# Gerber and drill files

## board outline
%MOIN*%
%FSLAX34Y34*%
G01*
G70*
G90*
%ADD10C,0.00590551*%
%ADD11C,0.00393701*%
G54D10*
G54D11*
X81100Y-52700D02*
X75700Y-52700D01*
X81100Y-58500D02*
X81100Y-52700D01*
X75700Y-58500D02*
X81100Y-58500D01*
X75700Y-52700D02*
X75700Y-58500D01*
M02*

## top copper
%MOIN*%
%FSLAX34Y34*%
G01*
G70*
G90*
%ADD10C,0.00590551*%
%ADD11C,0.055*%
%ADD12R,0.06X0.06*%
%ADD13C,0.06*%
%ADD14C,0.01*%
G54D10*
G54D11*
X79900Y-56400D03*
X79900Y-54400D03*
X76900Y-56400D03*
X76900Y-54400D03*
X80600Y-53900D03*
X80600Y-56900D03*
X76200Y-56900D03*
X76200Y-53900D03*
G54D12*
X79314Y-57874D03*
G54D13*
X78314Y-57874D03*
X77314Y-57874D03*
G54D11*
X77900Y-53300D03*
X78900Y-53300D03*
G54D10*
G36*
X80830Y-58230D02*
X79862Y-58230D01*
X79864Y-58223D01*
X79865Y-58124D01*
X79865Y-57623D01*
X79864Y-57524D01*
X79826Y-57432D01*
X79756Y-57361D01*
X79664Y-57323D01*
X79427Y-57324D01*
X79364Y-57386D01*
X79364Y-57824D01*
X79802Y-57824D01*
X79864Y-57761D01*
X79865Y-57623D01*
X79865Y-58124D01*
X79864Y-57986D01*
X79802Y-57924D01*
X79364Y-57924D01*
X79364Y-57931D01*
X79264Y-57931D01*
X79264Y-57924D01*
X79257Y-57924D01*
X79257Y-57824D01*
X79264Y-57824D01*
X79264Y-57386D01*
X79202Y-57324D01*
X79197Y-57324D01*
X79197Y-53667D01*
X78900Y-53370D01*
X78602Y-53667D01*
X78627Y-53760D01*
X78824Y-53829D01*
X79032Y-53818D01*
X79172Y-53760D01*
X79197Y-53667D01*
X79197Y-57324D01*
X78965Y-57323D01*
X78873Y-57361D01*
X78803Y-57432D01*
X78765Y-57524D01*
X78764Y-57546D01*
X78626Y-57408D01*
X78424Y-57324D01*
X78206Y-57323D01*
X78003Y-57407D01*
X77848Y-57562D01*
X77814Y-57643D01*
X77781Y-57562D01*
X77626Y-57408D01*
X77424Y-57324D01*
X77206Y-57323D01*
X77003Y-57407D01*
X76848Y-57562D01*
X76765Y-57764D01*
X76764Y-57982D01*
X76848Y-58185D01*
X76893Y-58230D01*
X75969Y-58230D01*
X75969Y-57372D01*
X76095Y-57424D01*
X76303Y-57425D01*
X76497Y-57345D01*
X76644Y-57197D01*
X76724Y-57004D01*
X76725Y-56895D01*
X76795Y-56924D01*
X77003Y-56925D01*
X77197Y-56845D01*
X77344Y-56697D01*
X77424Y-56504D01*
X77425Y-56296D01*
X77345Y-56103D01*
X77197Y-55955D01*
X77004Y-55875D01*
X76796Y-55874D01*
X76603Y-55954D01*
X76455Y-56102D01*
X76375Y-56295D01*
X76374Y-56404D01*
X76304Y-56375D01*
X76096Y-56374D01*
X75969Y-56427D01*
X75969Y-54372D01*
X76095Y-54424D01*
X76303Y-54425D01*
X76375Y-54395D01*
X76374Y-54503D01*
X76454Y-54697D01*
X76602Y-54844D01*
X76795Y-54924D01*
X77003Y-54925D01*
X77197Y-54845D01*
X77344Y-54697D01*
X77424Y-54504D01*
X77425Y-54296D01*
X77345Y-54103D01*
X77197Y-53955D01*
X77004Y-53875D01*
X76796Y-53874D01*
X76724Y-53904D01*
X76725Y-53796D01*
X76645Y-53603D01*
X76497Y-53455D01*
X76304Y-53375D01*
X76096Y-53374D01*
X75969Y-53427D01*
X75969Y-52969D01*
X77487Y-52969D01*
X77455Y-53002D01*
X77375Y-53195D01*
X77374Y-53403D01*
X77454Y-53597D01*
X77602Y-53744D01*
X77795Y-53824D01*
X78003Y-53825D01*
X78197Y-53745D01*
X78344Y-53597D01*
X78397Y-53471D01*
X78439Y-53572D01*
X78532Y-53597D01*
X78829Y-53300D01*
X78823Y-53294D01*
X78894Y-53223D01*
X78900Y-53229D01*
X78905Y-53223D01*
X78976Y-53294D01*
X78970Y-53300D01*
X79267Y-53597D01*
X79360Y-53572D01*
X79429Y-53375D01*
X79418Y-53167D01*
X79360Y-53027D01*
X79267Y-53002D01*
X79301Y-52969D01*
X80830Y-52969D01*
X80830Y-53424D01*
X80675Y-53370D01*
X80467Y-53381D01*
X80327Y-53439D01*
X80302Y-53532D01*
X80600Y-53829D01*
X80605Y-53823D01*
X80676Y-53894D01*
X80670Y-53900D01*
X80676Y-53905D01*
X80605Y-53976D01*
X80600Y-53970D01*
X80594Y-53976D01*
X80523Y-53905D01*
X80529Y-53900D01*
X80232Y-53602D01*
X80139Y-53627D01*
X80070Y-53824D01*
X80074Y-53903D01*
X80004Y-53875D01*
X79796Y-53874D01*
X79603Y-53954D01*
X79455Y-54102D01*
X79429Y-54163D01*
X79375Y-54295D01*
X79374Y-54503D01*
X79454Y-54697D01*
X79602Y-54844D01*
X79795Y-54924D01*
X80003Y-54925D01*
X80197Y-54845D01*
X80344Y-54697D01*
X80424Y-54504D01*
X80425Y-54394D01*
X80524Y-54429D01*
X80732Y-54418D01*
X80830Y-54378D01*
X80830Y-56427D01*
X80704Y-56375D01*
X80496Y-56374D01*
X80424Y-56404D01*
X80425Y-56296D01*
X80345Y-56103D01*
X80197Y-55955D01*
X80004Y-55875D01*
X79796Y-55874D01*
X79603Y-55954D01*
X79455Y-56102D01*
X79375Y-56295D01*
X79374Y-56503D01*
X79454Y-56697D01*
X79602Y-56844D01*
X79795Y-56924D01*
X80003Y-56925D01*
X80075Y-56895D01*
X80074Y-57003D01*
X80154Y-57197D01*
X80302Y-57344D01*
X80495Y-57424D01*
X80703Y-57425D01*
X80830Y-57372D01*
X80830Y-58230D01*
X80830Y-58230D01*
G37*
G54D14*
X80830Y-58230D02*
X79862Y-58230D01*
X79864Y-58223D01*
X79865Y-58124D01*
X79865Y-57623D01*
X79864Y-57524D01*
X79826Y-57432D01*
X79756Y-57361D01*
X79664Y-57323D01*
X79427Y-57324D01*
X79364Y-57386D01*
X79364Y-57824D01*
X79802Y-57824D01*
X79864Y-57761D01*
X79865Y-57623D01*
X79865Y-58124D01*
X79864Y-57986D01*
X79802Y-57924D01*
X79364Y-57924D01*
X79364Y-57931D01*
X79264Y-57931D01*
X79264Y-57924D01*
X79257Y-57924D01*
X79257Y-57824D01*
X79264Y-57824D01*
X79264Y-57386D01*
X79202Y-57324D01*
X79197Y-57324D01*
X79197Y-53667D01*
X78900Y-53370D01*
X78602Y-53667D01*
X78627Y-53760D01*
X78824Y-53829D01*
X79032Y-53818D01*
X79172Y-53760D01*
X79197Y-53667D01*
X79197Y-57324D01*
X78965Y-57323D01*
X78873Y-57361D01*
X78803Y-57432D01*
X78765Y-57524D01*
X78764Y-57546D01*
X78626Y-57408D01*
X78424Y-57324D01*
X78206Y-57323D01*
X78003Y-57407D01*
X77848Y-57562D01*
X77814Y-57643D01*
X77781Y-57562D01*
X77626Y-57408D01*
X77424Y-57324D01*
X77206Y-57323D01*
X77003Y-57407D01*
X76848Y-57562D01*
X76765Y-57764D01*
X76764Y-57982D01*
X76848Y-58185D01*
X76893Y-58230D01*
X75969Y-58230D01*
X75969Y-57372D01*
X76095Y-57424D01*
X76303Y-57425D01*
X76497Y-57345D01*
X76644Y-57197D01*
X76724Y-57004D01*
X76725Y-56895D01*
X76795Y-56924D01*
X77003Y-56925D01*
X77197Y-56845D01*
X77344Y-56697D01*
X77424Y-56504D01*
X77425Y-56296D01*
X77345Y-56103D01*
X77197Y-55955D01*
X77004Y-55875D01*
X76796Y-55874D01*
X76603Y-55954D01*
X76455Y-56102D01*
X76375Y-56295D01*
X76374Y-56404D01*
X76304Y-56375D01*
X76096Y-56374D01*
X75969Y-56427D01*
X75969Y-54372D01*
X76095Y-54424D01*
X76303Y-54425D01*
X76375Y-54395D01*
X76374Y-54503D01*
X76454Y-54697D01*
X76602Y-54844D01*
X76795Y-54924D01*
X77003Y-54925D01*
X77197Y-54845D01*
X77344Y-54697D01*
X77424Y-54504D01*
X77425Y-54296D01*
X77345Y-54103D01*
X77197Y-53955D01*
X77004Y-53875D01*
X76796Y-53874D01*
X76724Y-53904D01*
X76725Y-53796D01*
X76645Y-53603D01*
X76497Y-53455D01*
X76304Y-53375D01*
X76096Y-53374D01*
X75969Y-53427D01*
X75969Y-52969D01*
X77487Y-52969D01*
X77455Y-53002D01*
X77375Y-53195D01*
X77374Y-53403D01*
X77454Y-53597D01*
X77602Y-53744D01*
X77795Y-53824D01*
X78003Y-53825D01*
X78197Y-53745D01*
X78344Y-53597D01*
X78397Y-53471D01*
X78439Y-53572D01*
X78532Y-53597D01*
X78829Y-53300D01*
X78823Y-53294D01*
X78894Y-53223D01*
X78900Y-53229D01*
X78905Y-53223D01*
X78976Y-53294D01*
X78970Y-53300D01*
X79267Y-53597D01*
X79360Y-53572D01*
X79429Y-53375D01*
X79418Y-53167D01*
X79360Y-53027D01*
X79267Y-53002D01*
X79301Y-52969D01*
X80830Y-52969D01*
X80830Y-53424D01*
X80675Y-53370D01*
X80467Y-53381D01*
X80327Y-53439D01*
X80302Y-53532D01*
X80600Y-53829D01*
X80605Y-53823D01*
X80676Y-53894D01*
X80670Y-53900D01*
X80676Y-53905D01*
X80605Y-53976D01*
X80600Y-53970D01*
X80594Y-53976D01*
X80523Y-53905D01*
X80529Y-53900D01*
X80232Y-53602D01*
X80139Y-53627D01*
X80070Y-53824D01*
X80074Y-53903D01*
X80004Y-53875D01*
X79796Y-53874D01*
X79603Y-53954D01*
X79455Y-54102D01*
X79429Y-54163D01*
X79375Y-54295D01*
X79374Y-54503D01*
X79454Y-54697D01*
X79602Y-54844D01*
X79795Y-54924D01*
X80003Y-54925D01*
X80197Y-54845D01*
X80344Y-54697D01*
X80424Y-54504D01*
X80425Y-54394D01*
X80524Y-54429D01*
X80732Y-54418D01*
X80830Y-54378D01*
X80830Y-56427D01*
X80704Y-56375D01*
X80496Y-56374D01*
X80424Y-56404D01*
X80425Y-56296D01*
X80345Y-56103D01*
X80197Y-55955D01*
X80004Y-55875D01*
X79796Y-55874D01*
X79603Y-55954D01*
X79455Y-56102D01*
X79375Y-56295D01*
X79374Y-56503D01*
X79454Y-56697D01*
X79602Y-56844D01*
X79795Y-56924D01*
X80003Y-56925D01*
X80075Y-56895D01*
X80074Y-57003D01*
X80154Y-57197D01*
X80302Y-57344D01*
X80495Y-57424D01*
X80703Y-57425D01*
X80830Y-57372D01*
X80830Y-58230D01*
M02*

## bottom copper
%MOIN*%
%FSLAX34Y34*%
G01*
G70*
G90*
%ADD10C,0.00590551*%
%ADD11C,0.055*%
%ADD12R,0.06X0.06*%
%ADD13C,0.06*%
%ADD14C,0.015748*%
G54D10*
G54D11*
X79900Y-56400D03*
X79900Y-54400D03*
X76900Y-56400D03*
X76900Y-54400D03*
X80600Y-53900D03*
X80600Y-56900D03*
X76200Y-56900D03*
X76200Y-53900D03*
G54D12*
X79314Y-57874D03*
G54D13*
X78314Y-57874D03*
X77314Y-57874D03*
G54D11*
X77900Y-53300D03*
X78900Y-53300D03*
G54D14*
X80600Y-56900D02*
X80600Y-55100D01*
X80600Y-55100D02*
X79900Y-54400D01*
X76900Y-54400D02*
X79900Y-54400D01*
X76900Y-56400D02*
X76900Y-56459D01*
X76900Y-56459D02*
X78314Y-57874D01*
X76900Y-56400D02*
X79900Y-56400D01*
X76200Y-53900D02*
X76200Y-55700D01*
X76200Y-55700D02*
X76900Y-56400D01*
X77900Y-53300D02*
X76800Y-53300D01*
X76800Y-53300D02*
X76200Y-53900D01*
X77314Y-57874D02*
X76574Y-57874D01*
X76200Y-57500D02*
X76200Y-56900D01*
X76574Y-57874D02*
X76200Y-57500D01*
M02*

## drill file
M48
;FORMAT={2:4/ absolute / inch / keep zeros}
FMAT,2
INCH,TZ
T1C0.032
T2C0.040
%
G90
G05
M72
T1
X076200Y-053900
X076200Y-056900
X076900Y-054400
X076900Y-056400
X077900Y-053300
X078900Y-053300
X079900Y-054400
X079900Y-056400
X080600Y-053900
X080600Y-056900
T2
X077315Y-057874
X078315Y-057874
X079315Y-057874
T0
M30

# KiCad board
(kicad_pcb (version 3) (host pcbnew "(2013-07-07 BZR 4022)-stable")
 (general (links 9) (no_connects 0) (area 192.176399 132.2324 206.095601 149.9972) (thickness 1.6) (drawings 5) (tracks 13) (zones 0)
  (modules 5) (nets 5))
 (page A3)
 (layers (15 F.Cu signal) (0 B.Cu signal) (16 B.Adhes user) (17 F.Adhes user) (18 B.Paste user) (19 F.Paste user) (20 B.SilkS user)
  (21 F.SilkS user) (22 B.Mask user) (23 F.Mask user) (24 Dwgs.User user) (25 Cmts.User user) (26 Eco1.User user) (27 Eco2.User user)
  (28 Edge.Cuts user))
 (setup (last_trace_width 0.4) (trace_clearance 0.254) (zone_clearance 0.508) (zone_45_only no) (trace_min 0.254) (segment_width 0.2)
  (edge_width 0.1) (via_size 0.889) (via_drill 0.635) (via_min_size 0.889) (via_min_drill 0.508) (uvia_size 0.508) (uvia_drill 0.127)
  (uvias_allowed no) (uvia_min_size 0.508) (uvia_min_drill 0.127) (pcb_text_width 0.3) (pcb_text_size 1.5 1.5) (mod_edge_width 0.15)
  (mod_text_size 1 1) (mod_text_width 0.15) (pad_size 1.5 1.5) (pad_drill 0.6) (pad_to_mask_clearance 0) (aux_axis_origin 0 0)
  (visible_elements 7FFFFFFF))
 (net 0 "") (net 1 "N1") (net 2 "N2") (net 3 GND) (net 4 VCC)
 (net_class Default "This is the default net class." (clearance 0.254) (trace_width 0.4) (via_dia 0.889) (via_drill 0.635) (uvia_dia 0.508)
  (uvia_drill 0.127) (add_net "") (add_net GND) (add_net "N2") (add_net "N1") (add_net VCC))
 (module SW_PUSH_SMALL (layer B.Cu) (at 199.136 140.716)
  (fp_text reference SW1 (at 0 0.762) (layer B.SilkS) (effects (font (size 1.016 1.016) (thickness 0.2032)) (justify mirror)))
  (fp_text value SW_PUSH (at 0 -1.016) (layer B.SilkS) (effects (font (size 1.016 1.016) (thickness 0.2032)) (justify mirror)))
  (pad 1 thru_hole circle (at 3.81 2.54) (size 1.397 1.397) (drill 0.8128) (layers *.Cu *.Mask B.SilkS) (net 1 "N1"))
  (pad 2 thru_hole circle (at 3.81 -2.54) (size 1.397 1.397) (drill 0.8128) (layers *.Cu *.Mask B.SilkS) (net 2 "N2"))
  (pad 1 thru_hole circle (at -3.81 2.54) (size 1.397 1.397) (drill 0.8128) (layers *.Cu *.Mask B.SilkS) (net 1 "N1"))
  (pad 2 thru_hole circle (at -3.81 -2.54) (size 1.397 1.397) (drill 0.8128) (layers *.Cu *.Mask B.SilkS) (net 2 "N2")))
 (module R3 (layer F.Cu) (at 204.724 140.716 270) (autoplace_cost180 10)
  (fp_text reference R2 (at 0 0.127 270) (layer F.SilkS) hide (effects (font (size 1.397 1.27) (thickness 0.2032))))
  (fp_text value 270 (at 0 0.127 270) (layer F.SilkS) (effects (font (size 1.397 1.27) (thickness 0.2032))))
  (pad 1 thru_hole circle (at -3.81 0 270) (size 1.397 1.397) (drill 0.8128) (layers *.Cu *.Mask F.SilkS) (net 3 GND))
  (pad 2 thru_hole circle (at 3.81 0 270) (size 1.397 1.397) (drill 0.8128) (layers *.Cu *.Mask F.SilkS) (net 2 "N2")))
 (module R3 (layer F.Cu) (at 193.548 140.716 90) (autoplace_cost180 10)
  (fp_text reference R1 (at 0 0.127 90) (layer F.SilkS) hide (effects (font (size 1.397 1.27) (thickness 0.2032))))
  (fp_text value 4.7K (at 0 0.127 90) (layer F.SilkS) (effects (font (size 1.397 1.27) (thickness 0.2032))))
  (pad 1 thru_hole circle (at -3.81 0 90) (size 1.397 1.397) (drill 0.8128) (layers *.Cu *.Mask F.SilkS) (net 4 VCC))
  (pad 2 thru_hole circle (at 3.81 0 90) (size 1.397 1.397) (drill 0.8128) (layers *.Cu *.Mask F.SilkS) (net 1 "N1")))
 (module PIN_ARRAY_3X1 (layer F.Cu) (at 198.92 147 180)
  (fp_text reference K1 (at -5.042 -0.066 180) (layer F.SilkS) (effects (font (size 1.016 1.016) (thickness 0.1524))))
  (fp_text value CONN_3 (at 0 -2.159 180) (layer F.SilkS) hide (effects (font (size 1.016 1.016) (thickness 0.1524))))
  (pad 1 thru_hole rect (at -2.54 0 180) (size 1.524 1.524) (drill 1.016) (layers *.Cu *.Mask F.SilkS) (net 3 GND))
  (pad 2 thru_hole circle (at 0 0 180) (size 1.524 1.524) (drill 1.016) (layers *.Cu *.Mask F.SilkS) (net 1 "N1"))
  (pad 3 thru_hole circle (at 2.54 0 180) (size 1.524 1.524) (drill 1.016) (layers *.Cu *.Mask F.SilkS) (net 4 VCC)))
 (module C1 (layer F.Cu) (at 199.136 135.382)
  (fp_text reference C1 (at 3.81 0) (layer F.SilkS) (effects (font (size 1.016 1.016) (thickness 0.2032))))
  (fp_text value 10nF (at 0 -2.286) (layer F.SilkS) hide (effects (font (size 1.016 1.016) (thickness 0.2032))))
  (pad 1 thru_hole circle (at -1.27 0) (size 1.397 1.397) (drill 0.8128) (layers *.Cu *.Mask F.SilkS) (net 1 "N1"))
  (pad 2 thru_hole circle (at 1.27 0) (size 1.397 1.397) (drill 0.8128) (layers *.Cu *.Mask F.SilkS) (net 3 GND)))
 (gr_line (start 205.994 133.858) (end 192.278 133.858) (angle 90) (layer Edge.Cuts) (width 0.1))
 (gr_line (start 205.994 148.59) (end 205.994 133.858) (angle 90) (layer Edge.Cuts) (width 0.1))
 (gr_line (start 192.278 148.59) (end 205.994 148.59) (angle 90) (layer Edge.Cuts) (width 0.1))
 (gr_line (start 192.278 133.858) (end 192.278 148.59) (angle 90) (layer Edge.Cuts) (width 0.1))
 (segment (start 204.724 144.526) (end 204.724 139.954) (width 0.4) (layer B.Cu) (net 2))
 (segment (start 204.724 139.954) (end 202.946 138.176) (width 0.4) (layer B.Cu) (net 2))
 (segment (start 195.326 138.176) (end 202.946 138.176) (width 0.4) (layer B.Cu) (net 2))
 (segment (start 195.326 143.256) (end 195.326 143.406) (width 0.4) (layer B.Cu) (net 1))
 (segment (start 195.326 143.406) (end 198.92 147) (width 0.4) (layer B.Cu) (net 1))
 (segment (start 195.326 143.256) (end 202.946 143.256) (width 0.4) (layer B.Cu) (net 1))
 (segment (start 193.548 136.906) (end 193.548 141.478) (width 0.4) (layer B.Cu) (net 1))
 (segment (start 193.548 141.478) (end 195.326 143.256) (width 0.4) (layer B.Cu) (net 1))
 (segment (start 197.866 135.382) (end 195.072 135.382) (width 0.4) (layer B.Cu) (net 1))
 (segment (start 195.072 135.382) (end 193.548 136.906) (width 0.4) (layer B.Cu) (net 1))
 (segment (start 196.38 147) (end 194.498 147) (width 0.4) (layer B.Cu) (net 4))
 (segment (start 193.548 146.05) (end 193.548 144.526) (width 0.4) (layer B.Cu) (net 4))
 (segment (start 194.498 147) (end 193.548 146.05) (width 0.4) (layer B.Cu) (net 4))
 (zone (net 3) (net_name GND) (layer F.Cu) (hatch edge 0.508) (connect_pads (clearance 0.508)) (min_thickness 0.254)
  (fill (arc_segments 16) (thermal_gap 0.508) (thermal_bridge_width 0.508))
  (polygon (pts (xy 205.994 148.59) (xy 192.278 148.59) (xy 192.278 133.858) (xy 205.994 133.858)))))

